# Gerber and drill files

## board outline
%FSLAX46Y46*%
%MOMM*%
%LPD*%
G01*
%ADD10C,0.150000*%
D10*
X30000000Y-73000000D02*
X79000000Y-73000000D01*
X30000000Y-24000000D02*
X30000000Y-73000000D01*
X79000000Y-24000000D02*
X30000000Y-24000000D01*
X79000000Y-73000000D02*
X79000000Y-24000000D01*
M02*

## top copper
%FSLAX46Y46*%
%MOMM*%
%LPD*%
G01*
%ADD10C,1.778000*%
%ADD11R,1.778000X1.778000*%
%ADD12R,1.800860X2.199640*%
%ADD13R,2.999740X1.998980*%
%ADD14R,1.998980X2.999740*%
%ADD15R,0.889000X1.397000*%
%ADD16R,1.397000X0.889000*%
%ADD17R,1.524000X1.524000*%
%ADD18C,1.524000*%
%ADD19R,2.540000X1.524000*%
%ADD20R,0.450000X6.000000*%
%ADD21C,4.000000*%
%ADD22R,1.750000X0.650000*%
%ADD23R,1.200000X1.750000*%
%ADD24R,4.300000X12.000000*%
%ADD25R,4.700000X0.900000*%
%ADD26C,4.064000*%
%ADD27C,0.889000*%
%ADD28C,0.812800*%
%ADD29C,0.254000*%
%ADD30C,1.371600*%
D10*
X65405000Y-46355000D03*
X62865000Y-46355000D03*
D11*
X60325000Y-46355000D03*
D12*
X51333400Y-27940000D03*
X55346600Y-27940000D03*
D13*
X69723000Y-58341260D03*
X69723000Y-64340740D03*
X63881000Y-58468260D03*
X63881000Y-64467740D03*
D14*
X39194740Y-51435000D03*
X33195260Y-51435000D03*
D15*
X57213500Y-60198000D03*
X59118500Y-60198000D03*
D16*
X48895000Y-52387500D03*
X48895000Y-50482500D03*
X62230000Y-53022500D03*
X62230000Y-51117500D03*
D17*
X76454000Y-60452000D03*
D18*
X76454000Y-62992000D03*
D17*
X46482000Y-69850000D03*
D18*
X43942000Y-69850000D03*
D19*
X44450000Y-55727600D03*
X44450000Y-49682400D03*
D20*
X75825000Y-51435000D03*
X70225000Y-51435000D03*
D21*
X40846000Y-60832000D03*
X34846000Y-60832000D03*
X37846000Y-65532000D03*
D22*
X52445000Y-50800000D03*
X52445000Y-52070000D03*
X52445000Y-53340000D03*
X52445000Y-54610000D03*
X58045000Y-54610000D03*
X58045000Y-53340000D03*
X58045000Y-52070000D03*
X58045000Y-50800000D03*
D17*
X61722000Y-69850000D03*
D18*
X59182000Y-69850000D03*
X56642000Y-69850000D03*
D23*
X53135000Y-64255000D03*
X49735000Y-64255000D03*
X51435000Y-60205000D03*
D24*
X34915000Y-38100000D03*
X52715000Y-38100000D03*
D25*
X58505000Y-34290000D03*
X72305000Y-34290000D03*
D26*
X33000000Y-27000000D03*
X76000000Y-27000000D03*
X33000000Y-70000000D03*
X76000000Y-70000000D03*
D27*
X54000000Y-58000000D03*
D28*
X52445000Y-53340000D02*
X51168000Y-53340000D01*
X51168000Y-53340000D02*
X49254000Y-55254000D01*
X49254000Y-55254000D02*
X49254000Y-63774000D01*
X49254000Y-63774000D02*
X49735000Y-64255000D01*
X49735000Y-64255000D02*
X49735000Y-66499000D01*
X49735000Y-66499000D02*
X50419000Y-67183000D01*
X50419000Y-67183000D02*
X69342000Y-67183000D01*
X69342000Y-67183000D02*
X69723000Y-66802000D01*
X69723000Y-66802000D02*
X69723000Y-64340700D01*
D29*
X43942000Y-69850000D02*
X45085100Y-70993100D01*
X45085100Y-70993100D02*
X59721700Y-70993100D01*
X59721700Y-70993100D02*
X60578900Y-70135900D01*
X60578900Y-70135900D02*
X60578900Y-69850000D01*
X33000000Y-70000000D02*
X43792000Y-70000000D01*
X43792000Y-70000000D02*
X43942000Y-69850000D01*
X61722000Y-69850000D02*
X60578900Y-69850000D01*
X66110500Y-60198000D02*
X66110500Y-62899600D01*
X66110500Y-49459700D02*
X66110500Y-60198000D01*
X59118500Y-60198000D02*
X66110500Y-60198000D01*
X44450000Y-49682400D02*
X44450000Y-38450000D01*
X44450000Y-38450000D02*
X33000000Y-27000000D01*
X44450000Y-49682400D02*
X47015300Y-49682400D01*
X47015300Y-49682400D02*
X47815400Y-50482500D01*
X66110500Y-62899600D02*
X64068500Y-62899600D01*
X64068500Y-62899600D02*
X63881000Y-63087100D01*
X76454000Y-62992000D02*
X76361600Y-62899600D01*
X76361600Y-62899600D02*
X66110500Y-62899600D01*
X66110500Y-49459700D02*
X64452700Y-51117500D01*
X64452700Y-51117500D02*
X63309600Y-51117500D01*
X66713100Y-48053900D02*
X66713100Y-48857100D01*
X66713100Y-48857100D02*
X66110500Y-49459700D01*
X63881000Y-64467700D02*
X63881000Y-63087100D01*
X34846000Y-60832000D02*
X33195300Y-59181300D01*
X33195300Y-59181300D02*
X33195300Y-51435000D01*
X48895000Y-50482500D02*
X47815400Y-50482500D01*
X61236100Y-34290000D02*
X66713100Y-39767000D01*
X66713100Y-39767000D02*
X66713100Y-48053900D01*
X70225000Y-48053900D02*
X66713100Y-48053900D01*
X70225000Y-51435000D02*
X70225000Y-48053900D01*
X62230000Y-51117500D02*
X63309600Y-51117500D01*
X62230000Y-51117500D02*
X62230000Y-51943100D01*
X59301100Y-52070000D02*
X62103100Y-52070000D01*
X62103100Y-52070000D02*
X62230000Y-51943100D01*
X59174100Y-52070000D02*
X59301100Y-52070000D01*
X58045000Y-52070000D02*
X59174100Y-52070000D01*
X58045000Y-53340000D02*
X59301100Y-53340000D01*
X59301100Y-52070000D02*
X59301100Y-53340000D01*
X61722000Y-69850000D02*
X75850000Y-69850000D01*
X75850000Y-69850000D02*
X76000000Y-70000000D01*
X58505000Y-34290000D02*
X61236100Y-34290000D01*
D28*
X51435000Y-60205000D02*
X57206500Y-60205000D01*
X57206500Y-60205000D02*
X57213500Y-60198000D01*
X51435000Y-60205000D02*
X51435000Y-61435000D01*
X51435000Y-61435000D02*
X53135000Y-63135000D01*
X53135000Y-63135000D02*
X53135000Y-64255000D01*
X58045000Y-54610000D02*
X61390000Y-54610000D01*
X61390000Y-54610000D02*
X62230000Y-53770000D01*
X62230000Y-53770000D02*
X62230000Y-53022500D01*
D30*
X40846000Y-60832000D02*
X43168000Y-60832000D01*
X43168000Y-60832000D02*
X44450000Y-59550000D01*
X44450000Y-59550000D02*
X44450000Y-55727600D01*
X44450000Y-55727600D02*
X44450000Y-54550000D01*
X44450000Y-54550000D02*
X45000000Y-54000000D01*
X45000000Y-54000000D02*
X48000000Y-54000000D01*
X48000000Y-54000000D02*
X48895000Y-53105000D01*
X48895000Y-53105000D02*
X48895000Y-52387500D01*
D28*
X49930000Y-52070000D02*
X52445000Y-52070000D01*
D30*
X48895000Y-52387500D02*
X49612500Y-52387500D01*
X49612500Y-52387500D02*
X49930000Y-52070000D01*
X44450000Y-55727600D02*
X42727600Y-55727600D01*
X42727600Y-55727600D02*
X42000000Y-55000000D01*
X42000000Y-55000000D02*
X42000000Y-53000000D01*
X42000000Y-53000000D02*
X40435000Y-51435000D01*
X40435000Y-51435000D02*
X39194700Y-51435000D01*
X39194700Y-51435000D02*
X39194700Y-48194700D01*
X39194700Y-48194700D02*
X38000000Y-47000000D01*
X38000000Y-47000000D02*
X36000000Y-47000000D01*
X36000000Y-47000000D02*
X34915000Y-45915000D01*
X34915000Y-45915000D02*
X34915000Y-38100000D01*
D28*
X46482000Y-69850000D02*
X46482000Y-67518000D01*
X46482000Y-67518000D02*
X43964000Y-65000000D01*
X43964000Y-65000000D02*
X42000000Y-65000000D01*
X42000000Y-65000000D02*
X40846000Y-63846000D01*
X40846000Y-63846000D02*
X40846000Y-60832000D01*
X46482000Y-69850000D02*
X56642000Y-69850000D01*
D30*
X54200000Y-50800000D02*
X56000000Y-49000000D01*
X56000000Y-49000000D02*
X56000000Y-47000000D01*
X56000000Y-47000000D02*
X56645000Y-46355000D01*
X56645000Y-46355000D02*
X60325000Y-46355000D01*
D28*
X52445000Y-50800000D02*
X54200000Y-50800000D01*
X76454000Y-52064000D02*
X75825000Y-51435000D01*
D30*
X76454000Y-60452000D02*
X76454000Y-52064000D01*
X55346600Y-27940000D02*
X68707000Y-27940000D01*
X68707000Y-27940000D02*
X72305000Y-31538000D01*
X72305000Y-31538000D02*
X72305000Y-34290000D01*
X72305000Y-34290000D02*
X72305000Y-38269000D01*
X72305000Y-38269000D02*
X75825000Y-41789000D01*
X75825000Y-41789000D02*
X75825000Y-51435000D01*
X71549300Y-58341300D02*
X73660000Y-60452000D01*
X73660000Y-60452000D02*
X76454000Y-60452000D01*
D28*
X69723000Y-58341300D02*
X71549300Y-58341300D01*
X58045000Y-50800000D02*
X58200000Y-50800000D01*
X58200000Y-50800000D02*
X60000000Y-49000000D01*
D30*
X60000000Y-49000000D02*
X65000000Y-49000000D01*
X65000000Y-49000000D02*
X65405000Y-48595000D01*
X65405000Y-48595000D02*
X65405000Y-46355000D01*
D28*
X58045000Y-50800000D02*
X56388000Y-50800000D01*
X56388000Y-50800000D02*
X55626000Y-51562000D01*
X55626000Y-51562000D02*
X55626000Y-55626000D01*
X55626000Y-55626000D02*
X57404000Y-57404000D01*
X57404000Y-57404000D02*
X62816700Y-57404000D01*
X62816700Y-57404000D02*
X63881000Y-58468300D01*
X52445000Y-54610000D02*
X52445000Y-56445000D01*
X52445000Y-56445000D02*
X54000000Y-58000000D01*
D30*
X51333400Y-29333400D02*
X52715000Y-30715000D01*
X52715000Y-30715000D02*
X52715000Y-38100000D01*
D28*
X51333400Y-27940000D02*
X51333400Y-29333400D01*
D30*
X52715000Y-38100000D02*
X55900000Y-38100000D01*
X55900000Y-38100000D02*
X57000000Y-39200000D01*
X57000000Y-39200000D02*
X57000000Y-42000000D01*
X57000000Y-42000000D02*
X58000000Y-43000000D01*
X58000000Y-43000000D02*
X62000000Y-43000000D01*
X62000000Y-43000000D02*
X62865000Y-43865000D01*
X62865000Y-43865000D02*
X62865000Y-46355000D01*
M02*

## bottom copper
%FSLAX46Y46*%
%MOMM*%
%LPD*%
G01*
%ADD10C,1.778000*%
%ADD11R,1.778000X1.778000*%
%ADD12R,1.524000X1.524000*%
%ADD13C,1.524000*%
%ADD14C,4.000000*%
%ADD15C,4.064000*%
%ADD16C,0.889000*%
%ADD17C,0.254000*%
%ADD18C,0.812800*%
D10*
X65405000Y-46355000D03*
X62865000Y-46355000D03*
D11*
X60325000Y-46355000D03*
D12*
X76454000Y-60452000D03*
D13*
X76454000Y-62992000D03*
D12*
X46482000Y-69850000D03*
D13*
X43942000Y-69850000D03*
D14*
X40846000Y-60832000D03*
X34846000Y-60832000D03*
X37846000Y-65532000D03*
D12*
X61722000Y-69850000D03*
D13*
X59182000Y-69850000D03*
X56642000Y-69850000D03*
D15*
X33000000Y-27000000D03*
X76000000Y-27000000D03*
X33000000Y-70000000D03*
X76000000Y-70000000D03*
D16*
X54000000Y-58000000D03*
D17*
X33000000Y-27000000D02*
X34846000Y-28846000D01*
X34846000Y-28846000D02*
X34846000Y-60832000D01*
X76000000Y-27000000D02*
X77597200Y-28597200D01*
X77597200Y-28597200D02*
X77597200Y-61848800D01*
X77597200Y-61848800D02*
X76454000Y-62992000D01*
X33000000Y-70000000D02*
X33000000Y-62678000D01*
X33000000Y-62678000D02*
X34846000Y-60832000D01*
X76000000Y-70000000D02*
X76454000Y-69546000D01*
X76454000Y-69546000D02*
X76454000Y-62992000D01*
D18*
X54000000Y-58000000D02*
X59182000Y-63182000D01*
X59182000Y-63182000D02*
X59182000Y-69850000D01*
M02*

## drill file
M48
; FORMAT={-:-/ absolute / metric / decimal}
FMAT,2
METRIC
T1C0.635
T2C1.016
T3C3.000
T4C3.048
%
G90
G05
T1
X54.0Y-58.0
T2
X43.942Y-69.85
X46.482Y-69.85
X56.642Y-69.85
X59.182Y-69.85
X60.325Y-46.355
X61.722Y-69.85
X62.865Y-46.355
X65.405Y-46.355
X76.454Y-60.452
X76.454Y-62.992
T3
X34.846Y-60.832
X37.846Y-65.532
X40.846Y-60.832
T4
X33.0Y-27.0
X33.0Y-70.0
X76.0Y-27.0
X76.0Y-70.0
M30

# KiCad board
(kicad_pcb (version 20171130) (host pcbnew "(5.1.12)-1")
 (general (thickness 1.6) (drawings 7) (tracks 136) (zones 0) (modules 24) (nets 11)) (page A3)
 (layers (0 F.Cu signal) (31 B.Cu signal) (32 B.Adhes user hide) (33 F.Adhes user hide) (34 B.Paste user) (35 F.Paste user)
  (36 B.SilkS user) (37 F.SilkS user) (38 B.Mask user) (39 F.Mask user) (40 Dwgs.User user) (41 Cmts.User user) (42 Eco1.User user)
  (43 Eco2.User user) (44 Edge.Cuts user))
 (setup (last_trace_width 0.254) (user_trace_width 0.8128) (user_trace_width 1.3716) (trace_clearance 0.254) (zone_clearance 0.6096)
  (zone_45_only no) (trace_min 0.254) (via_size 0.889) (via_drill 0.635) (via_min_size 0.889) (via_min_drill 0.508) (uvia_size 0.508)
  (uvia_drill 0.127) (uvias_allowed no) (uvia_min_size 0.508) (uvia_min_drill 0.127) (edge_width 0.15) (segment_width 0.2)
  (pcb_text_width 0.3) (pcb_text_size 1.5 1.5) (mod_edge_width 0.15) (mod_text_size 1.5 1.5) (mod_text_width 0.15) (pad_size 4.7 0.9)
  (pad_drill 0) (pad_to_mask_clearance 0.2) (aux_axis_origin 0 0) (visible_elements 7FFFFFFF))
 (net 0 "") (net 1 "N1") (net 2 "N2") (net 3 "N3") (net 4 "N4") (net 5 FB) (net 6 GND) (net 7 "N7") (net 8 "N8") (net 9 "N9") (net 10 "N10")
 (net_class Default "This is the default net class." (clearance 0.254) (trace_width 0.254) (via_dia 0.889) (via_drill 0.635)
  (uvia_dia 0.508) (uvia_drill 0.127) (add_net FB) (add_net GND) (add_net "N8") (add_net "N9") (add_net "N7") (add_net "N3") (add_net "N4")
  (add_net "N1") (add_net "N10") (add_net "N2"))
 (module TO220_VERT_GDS (layer F.Cu) (at 62.865 46.355 270)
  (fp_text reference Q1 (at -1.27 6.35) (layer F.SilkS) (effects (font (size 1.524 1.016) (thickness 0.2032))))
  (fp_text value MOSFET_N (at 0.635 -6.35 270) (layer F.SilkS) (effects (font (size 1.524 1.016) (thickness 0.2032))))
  (pad S thru_hole circle (at 0 -2.54 270) (size 1.778 1.778) (drill 1.016) (layers *.Cu *.Mask F.SilkS) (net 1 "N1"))
  (pad D thru_hole circle (at 0 0 270) (size 1.778 1.778) (drill 1.016) (layers *.Cu *.Mask F.SilkS) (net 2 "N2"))
  (pad G thru_hole rect (at 0 2.54 270) (size 1.778 1.778) (drill 1.016) (layers *.Cu *.Mask F.SilkS) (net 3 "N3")))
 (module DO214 (layer F.Cu) (at 53.34 27.94)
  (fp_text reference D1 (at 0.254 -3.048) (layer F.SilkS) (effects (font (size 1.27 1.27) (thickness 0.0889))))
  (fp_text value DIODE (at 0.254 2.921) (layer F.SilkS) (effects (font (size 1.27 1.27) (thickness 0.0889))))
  (pad 1 smd rect (at -2.0066 0) (size 1.80086 2.19964) (layers F.Cu F.Paste F.Mask) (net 2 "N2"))
  (pad 2 smd rect (at 2.0066 0) (size 1.80086 2.19964) (layers F.Cu F.Paste F.Mask) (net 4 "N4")))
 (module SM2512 (layer F.Cu) (at 69.723 61.341 270)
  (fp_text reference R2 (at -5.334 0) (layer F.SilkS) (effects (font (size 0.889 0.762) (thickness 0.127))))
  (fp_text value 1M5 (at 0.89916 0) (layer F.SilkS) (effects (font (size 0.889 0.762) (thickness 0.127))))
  (pad 1 smd rect (at -2.99974 0 270) (size 1.99898 2.99974) (layers F.Cu F.Paste F.Mask) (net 4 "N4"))
  (pad 2 smd rect (at 2.99974 0 270) (size 1.99898 2.99974) (layers F.Cu F.Paste F.Mask) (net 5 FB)))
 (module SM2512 (layer F.Cu) (at 63.881 61.468 270)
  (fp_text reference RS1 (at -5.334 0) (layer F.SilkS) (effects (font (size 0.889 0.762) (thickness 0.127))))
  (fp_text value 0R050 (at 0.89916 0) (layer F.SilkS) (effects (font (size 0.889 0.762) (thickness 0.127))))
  (pad 1 smd rect (at -2.99974 0 270) (size 1.99898 2.99974) (layers F.Cu F.Paste F.Mask) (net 1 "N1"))
  (pad 2 smd rect (at 2.99974 0 270) (size 1.99898 2.99974) (layers F.Cu F.Paste F.Mask) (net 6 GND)))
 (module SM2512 (layer F.Cu) (at 36.195 51.435 180)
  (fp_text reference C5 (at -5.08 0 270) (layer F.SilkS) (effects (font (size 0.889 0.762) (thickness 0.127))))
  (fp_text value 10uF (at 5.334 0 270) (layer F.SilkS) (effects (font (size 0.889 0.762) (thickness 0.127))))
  (pad 1 smd rect (at -2.99974 0 180) (size 1.99898 2.99974) (layers F.Cu F.Paste F.Mask) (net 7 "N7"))
  (pad 2 smd rect (at 2.99974 0 180) (size 1.99898 2.99974) (layers F.Cu F.Paste F.Mask) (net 6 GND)))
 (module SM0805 (layer F.Cu) (at 58.166 60.198)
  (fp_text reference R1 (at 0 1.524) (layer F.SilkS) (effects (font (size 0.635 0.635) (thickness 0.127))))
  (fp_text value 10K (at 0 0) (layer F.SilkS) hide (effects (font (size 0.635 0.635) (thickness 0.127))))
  (pad 1 smd rect (at -0.9525 0) (size 0.889 1.397) (layers F.Cu F.Paste F.Mask) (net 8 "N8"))
  (pad 2 smd rect (at 0.9525 0) (size 0.889 1.397) (layers F.Cu F.Paste F.Mask) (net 6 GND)))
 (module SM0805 (layer F.Cu) (at 48.895 51.435 90)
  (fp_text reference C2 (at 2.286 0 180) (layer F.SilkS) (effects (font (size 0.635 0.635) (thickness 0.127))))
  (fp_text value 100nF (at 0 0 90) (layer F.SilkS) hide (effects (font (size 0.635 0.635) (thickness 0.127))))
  (pad 1 smd rect (at -0.9525 0 90) (size 0.889 1.397) (layers F.Cu F.Paste F.Mask) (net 7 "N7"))
  (pad 2 smd rect (at 0.9525 0 90) (size 0.889 1.397) (layers F.Cu F.Paste F.Mask) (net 6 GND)))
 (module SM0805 (layer F.Cu) (at 62.23 52.07 90)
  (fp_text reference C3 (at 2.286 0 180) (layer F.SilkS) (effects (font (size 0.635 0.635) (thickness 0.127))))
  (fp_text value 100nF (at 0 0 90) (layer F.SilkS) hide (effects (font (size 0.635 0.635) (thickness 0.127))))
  (pad 1 smd rect (at -0.9525 0 90) (size 0.889 1.397) (layers F.Cu F.Paste F.Mask) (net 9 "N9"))
  (pad 2 smd rect (at 0.9525 0 90) (size 0.889 1.397) (layers F.Cu F.Paste F.Mask) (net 6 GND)))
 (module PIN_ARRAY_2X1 (layer F.Cu) (at 76.454 61.722 270)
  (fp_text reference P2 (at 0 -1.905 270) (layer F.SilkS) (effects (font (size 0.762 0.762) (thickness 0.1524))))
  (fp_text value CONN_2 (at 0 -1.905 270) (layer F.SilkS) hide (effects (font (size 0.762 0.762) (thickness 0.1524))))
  (pad 1 thru_hole rect (at -1.27 0 270) (size 1.524 1.524) (drill 1.016) (layers *.Cu *.Mask F.SilkS) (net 4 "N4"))
  (pad 2 thru_hole circle (at 1.27 0 270) (size 1.524 1.524) (drill 1.016) (layers *.Cu *.Mask F.SilkS) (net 6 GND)))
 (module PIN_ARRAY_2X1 (layer F.Cu) (at 45.212 69.85 180)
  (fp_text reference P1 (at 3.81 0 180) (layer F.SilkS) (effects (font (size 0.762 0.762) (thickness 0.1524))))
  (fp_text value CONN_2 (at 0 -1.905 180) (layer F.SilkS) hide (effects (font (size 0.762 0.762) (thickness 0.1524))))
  (pad 1 thru_hole rect (at -1.27 0 180) (size 1.524 1.524) (drill 1.016) (layers *.Cu *.Mask F.SilkS) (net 7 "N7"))
  (pad 2 thru_hole circle (at 1.27 0 180) (size 1.524 1.524) (drill 1.016) (layers *.Cu *.Mask F.SilkS) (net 6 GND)))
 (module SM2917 (layer F.Cu) (at 44.45 52.705 90)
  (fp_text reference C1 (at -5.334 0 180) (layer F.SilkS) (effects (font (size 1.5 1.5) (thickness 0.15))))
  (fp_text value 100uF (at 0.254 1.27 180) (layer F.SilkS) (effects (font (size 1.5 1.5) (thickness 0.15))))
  (pad 1 smd rect (at -3.0226 0 90) (size 1.524 2.54) (layers F.Cu F.Paste F.Mask) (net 7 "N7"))
  (pad 2 smd rect (at 3.0226 0 90) (size 1.524 2.54) (layers F.Cu F.Paste F.Mask) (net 6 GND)))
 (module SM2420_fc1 (layer F.Cu) (at 73.025 51.435 180)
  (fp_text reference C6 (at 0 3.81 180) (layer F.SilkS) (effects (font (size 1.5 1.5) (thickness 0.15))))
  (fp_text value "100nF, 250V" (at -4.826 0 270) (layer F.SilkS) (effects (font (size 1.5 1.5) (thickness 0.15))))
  (pad 1 smd rect (at -2.8 0 180) (size 0.45 6) (layers F.Cu F.Paste F.Mask) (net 4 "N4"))
  (pad 2 smd rect (at 2.8 0 180) (size 0.45 6) (layers F.Cu F.Paste F.Mask) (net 6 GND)))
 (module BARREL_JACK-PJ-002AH (layer F.Cu) (at 37.846 65.532 180)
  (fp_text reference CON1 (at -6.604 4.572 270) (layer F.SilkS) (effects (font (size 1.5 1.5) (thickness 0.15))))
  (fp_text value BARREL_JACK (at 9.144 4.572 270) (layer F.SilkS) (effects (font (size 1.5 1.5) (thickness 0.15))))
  (pad 1 thru_hole circle (at -3 4.7 180) (size 4 4) (drill 3) (layers *.Cu *.Mask F.SilkS) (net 7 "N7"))
  (pad 2 thru_hole circle (at 3 4.7 180) (size 4 4) (drill 3) (layers *.Cu *.Mask F.SilkS) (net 6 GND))
  (pad 3 thru_hole circle (at 0 0 180) (size 4 4) (drill 3) (layers *.Cu *.Mask F.SilkS)))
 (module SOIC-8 (layer F.Cu) (at 55.245 52.705 270)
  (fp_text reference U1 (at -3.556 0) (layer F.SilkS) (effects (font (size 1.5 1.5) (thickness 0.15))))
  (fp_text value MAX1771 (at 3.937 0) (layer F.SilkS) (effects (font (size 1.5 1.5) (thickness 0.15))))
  (pad 1 smd rect (at -1.905 2.8 270) (size 0.65 1.75) (layers F.Cu F.Paste F.Mask) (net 3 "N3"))
  (pad 2 smd rect (at -0.635 2.8 270) (size 0.65 1.75) (layers F.Cu F.Paste F.Mask) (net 7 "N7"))
  (pad 3 smd rect (at 0.635 2.8 270) (size 0.65 1.75) (layers F.Cu F.Paste F.Mask) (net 5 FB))
  (pad 4 smd rect (at 1.905 2.8 270) (size 0.65 1.75) (layers F.Cu F.Paste F.Mask) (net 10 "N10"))
  (pad 5 smd rect (at 1.905 -2.8 270) (size 0.65 1.75) (layers F.Cu F.Paste F.Mask) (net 9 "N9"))
  (pad 6 smd rect (at 0.635 -2.8 270) (size 0.65 1.75) (layers F.Cu F.Paste F.Mask) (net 6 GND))
  (pad 7 smd rect (at -0.635 -2.8 270) (size 0.65 1.75) (layers F.Cu F.Paste F.Mask) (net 6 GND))
  (pad 8 smd rect (at -1.905 -2.8 270) (size 0.65 1.75) (layers F.Cu F.Paste F.Mask) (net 1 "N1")))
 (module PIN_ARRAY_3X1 (layer F.Cu) (at 59.182 69.85 180)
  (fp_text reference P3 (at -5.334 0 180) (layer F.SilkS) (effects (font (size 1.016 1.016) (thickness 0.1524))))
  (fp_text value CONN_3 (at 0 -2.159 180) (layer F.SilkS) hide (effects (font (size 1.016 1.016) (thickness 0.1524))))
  (pad 1 thru_hole rect (at -2.54 0 180) (size 1.524 1.524) (drill 1.016) (layers *.Cu *.Mask F.SilkS) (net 6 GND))
  (pad 2 thru_hole circle (at 0 0 180) (size 1.524 1.524) (drill 1.016) (layers *.Cu *.Mask F.SilkS) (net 10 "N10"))
  (pad 3 thru_hole circle (at 2.54 0 180) (size 1.524 1.524) (drill 1.016) (layers *.Cu *.Mask F.SilkS) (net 7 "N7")))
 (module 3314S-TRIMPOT (layer F.Cu) (at 51.435 62.23 180)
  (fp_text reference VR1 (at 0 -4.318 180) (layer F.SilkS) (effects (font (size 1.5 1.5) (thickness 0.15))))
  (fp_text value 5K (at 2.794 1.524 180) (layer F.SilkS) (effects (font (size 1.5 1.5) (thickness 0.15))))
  (pad 3 smd rect (at -1.7 -2.025 180) (size 1.2 1.75) (layers F.Cu F.Paste F.Mask) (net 8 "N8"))
  (pad 1 smd rect (at 1.7 -2.025 180) (size 1.2 1.75) (layers F.Cu F.Paste F.Mask) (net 5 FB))
  (pad 2 smd rect (at 0 2.025 180) (size 1.2 1.75) (layers F.Cu F.Paste F.Mask) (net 8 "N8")))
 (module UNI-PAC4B (layer F.Cu) (at 43.815 38.1)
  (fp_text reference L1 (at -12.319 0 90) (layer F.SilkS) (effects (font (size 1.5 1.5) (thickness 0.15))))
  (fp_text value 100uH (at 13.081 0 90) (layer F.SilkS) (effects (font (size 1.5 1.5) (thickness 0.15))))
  (pad 1 smd rect (at -8.9 0) (size 4.3 12) (layers F.Cu F.Paste F.Mask) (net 7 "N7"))
  (pad 2 smd rect (at 8.9 0) (size 4.3 12) (layers F.Cu F.Paste F.Mask) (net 2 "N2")))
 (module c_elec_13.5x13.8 (layer F.Cu) (at 65.405 34.29)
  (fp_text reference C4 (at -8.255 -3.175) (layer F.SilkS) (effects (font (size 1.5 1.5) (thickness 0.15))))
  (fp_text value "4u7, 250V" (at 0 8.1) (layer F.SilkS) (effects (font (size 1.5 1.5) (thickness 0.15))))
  (pad 2 smd rect (at -6.9 0) (size 4.7 0.9) (layers F.Cu F.Paste F.Mask) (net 6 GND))
  (pad 1 smd rect (at 6.9 0) (size 4.7 0.9) (layers F.Cu F.Paste F.Mask) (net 4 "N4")))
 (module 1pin (layer F.Cu) (at 33 27)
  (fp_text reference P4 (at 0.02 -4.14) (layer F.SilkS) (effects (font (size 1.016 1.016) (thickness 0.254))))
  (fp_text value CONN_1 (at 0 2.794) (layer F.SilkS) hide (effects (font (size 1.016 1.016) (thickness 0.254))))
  (pad 1 thru_hole circle (at 0 0) (size 4.064 4.064) (drill 3.048) (layers *.Cu *.Mask F.SilkS) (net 6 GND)))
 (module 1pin (layer F.Cu) (at 76 27)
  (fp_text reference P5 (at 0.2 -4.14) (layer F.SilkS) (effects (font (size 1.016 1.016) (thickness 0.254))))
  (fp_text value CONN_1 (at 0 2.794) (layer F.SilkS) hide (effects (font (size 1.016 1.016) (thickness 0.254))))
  (pad 1 thru_hole circle (at 0 0) (size 4.064 4.064) (drill 3.048) (layers *.Cu *.Mask F.SilkS) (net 6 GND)))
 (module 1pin (layer F.Cu) (at 33 70)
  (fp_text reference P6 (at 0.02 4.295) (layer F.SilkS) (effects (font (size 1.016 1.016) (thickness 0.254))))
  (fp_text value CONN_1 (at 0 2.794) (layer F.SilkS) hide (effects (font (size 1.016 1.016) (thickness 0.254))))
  (pad 1 thru_hole circle (at 0 0) (size 4.064 4.064) (drill 3.048) (layers *.Cu *.Mask F.SilkS) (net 6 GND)))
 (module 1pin (layer F.Cu) (at 76 70)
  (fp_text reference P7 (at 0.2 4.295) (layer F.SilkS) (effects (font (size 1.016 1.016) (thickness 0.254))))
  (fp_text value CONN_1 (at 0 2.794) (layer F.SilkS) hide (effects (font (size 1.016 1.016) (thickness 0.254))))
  (pad 1 thru_hole circle (at 0 0) (size 4.064 4.064) (drill 3.048) (layers *.Cu *.Mask F.SilkS) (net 6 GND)))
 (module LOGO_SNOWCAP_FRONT (layer F.Cu) (at 53 65)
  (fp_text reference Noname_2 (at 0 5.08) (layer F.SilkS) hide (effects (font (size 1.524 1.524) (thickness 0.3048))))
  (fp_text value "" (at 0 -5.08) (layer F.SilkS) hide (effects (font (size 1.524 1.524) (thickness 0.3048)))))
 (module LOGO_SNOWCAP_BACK (layer B.Cu) (at 53 51)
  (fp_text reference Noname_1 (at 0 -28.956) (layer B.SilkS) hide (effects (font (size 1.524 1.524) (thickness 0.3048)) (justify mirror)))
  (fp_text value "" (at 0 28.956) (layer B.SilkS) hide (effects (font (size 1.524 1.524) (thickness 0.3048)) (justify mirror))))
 (gr_line (start 30 73) (end 79 73) (angle 90) (layer Edge.Cuts) (width 0.15))
 (gr_line (start 30 24) (end 30 73) (angle 90) (layer Edge.Cuts) (width 0.15))
 (gr_line (start 79 24) (end 30 24) (angle 90) (layer Edge.Cuts) (width 0.15))
 (gr_line (start 79 73) (end 79 24) (angle 90) (layer Edge.Cuts) (width 0.15))
 (segment (start 52.445 53.34) (end 51.168 53.34) (width 0.8128) (layer F.Cu) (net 5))
 (segment (start 51.168 53.34) (end 49.254 55.254) (width 0.8128) (layer F.Cu) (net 5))
 (segment (start 49.254 55.254) (end 49.254 63.774) (width 0.8128) (layer F.Cu) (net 5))
 (segment (start 49.254 63.774) (end 49.735 64.255) (width 0.8128) (layer F.Cu) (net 5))
 (segment (start 49.735 64.255) (end 49.735 66.499) (width 0.8128) (layer F.Cu) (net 5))
 (segment (start 49.735 66.499) (end 50.419 67.183) (width 0.8128) (layer F.Cu) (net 5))
 (segment (start 50.419 67.183) (end 69.342 67.183) (width 0.8128) (layer F.Cu) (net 5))
 (segment (start 69.342 67.183) (end 69.723 66.802) (width 0.8128) (layer F.Cu) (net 5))
 (segment (start 69.723 66.802) (end 69.723 64.3407) (width 0.8128) (layer F.Cu) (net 5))
 (segment (start 43.942 69.85) (end 45.0851 70.9931) (width 0.254) (layer F.Cu) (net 6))
 (segment (start 45.0851 70.9931) (end 59.7217 70.9931) (width 0.254) (layer F.Cu) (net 6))
 (segment (start 59.7217 70.9931) (end 60.5789 70.1359) (width 0.254) (layer F.Cu) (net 6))
 (segment (start 60.5789 70.1359) (end 60.5789 69.85) (width 0.254) (layer F.Cu) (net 6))
 (segment (start 33 70) (end 43.792 70) (width 0.254) (layer F.Cu) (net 6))
 (segment (start 43.792 70) (end 43.942 69.85) (width 0.254) (layer F.Cu) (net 6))
 (segment (start 61.722 69.85) (end 60.5789 69.85) (width 0.254) (layer F.Cu) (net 6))
 (segment (start 66.1105 60.198) (end 66.1105 62.8996) (width 0.254) (layer F.Cu) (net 6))
 (segment (start 66.1105 49.4597) (end 66.1105 60.198) (width 0.254) (layer F.Cu) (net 6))
 (segment (start 59.1185 60.198) (end 66.1105 60.198) (width 0.254) (layer F.Cu) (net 6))
 (segment (start 44.45 49.6824) (end 44.45 38.45) (width 0.254) (layer F.Cu) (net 6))
 (segment (start 44.45 38.45) (end 33 27) (width 0.254) (layer F.Cu) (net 6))
 (segment (start 44.45 49.6824) (end 47.0153 49.6824) (width 0.254) (layer F.Cu) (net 6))
 (segment (start 47.0153 49.6824) (end 47.8154 50.4825) (width 0.254) (layer F.Cu) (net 6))
 (segment (start 66.1105 62.8996) (end 64.0685 62.8996) (width 0.254) (layer F.Cu) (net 6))
 (segment (start 64.0685 62.8996) (end 63.881 63.0871) (width 0.254) (layer F.Cu) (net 6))
 (segment (start 76.454 62.992) (end 76.3616 62.8996) (width 0.254) (layer F.Cu) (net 6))
 (segment (start 76.3616 62.8996) (end 66.1105 62.8996) (width 0.254) (layer F.Cu) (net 6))
 (segment (start 66.1105 49.4597) (end 64.4527 51.1175) (width 0.254) (layer F.Cu) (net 6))
 (segment (start 64.4527 51.1175) (end 63.3096 51.1175) (width 0.254) (layer F.Cu) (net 6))
 (segment (start 66.7131 48.0539) (end 66.7131 48.8571) (width 0.254) (layer F.Cu) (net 6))
 (segment (start 66.7131 48.8571) (end 66.1105 49.4597) (width 0.254) (layer F.Cu) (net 6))
 (segment (start 63.881 64.4677) (end 63.881 63.0871) (width 0.254) (layer F.Cu) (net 6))
 (segment (start 34.846 60.832) (end 33.1953 59.1813) (width 0.254) (layer F.Cu) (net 6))
 (segment (start 33.1953 59.1813) (end 33.1953 51.435) (width 0.254) (layer F.Cu) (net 6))
 (segment (start 48.895 50.4825) (end 47.8154 50.4825) (width 0.254) (layer F.Cu) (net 6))
 (segment (start 61.2361 34.29) (end 66.7131 39.767) (width 0.254) (layer F.Cu) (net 6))
 (segment (start 66.7131 39.767) (end 66.7131 48.0539) (width 0.254) (layer F.Cu) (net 6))
 (segment (start 70.225 48.0539) (end 66.7131 48.0539) (width 0.254) (layer F.Cu) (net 6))
 (segment (start 70.225 51.435) (end 70.225 48.0539) (width 0.254) (layer F.Cu) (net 6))
 (segment (start 62.23 51.1175) (end 63.3096 51.1175) (width 0.254) (layer F.Cu) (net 6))
 (segment (start 62.23 51.1175) (end 62.23 51.9431) (width 0.254) (layer F.Cu) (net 6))
 (segment (start 59.3011 52.07) (end 62.1031 52.07) (width 0.254) (layer F.Cu) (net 6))
 (segment (start 62.1031 52.07) (end 62.23 51.9431) (width 0.254) (layer F.Cu) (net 6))
 (segment (start 59.1741 52.07) (end 59.3011 52.07) (width 0.254) (layer F.Cu) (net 6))
 (segment (start 58.045 52.07) (end 59.1741 52.07) (width 0.254) (layer F.Cu) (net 6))
 (segment (start 58.045 53.34) (end 59.3011 53.34) (width 0.254) (layer F.Cu) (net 6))
 (segment (start 59.3011 52.07) (end 59.3011 53.34) (width 0.254) (layer F.Cu) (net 6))
 (segment (start 61.722 69.85) (end 75.85 69.85) (width 0.254) (layer F.Cu) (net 6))
 (segment (start 75.85 69.85) (end 76 70) (width 0.254) (layer F.Cu) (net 6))
 (segment (start 58.505 34.29) (end 61.2361 34.29) (width 0.254) (layer F.Cu) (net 6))
 (segment (start 33 27) (end 34.846 28.846) (width 0.254) (layer B.Cu) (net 6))
 (segment (start 34.846 28.846) (end 34.846 60.832) (width 0.254) (layer B.Cu) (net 6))
 (segment (start 76 27) (end 77.5972 28.5972) (width 0.254) (layer B.Cu) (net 6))
 (segment (start 77.5972 28.5972) (end 77.5972 61.8488) (width 0.254) (layer B.Cu) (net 6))
 (segment (start 77.5972 61.8488) (end 76.454 62.992) (width 0.254) (layer B.Cu) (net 6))
 (segment (start 33 70) (end 33 62.678) (width 0.254) (layer B.Cu) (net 6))
 (segment (start 33 62.678) (end 34.846 60.832) (width 0.254) (layer B.Cu) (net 6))
 (segment (start 76 70) (end 76.454 69.546) (width 0.254) (layer B.Cu) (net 6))
 (segment (start 76.454 69.546) (end 76.454 62.992) (width 0.254) (layer B.Cu) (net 6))
 (segment (start 51.435 60.205) (end 57.2065 60.205) (width 0.8128) (layer F.Cu) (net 8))
 (segment (start 57.2065 60.205) (end 57.2135 60.198) (width 0.8128) (layer F.Cu) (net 8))
 (segment (start 51.435 60.205) (end 51.435 61.435) (width 0.8128) (layer F.Cu) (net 8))
 (segment (start 51.435 61.435) (end 53.135 63.135) (width 0.8128) (layer F.Cu) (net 8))
 (segment (start 53.135 63.135) (end 53.135 64.255) (width 0.8128) (layer F.Cu) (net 8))
 (segment (start 58.045 54.61) (end 61.39 54.61) (width 0.8128) (layer F.Cu) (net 9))
 (segment (start 61.39 54.61) (end 62.23 53.77) (width 0.8128) (layer F.Cu) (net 9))
 (segment (start 62.23 53.77) (end 62.23 53.0225) (width 0.8128) (layer F.Cu) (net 9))
 (segment (start 40.846 60.832) (end 43.168 60.832) (width 1.3716) (layer F.Cu) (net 7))
 (segment (start 43.168 60.832) (end 44.45 59.55) (width 1.3716) (layer F.Cu) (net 7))
 (segment (start 44.45 59.55) (end 44.45 55.7276) (width 1.3716) (layer F.Cu) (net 7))
 (segment (start 44.45 55.7276) (end 44.45 54.55) (width 1.3716) (layer F.Cu) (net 7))
 (segment (start 44.45 54.55) (end 45 54) (width 1.3716) (layer F.Cu) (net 7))
 (segment (start 45 54) (end 48 54) (width 1.3716) (layer F.Cu) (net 7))
 (segment (start 48 54) (end 48.895 53.105) (width 1.3716) (layer F.Cu) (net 7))
 (segment (start 48.895 53.105) (end 48.895 52.3875) (width 1.3716) (layer F.Cu) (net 7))
 (segment (start 49.93 52.07) (end 52.445 52.07) (width 0.8128) (layer F.Cu) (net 7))
 (segment (start 48.895 52.3875) (end 49.6125 52.3875) (width 1.3716) (layer F.Cu) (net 7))
 (segment (start 49.6125 52.3875) (end 49.93 52.07) (width 1.3716) (layer F.Cu) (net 7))
 (segment (start 44.45 55.7276) (end 42.7276 55.7276) (width 1.3716) (layer F.Cu) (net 7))
 (segment (start 42.7276 55.7276) (end 42 55) (width 1.3716) (layer F.Cu) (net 7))
 (segment (start 42 55) (end 42 53) (width 1.3716) (layer F.Cu) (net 7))
 (segment (start 42 53) (end 40.435 51.435) (width 1.3716) (layer F.Cu) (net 7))
 (segment (start 40.435 51.435) (end 39.1947 51.435) (width 1.3716) (layer F.Cu) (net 7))
 (segment (start 39.1947 51.435) (end 39.1947 48.1947) (width 1.3716) (layer F.Cu) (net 7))
 (segment (start 39.1947 48.1947) (end 38 47) (width 1.3716) (layer F.Cu) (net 7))
 (segment (start 38 47) (end 36 47) (width 1.3716) (layer F.Cu) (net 7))
 (segment (start 36 47) (end 34.915 45.915) (width 1.3716) (layer F.Cu) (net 7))
 (segment (start 34.915 45.915) (end 34.915 38.1) (width 1.3716) (layer F.Cu) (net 7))
 (segment (start 46.482 69.85) (end 46.482 67.518) (width 0.8128) (layer F.Cu) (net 7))
 (segment (start 46.482 67.518) (end 43.964 65) (width 0.8128) (layer F.Cu) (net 7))
 (segment (start 43.964 65) (end 42 65) (width 0.8128) (layer F.Cu) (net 7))
 (segment (start 42 65) (end 40.846 63.846) (width 0.8128) (layer F.Cu) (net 7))
 (segment (start 40.846 63.846) (end 40.846 60.832) (width 0.8128) (layer F.Cu) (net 7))
 (segment (start 46.482 69.85) (end 56.642 69.85) (width 0.8128) (layer F.Cu) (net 7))
 (segment (start 54.2 50.8) (end 56 49) (width 1.3716) (layer F.Cu) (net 3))
 (segment (start 56 49) (end 56 47) (width 1.3716) (layer F.Cu) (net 3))
 (segment (start 56 47) (end 56.645 46.355) (width 1.3716) (layer F.Cu) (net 3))
 (segment (start 56.645 46.355) (end 60.325 46.355) (width 1.3716) (layer F.Cu) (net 3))
 (segment (start 52.445 50.8) (end 54.2 50.8) (width 0.8128) (layer F.Cu) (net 3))
 (segment (start 76.454 52.064) (end 75.825 51.435) (width 0.8128) (layer F.Cu) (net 4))
 (segment (start 76.454 60.452) (end 76.454 52.064) (width 1.3716) (layer F.Cu) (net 4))
 (segment (start 55.3466 27.94) (end 68.707 27.94) (width 1.3716) (layer F.Cu) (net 4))
 (segment (start 68.707 27.94) (end 72.305 31.538) (width 1.3716) (layer F.Cu) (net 4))
 (segment (start 72.305 31.538) (end 72.305 34.29) (width 1.3716) (layer F.Cu) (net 4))
 (segment (start 72.305 34.29) (end 72.305 38.269) (width 1.3716) (layer F.Cu) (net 4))
 (segment (start 72.305 38.269) (end 75.825 41.789) (width 1.3716) (layer F.Cu) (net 4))
 (segment (start 75.825 41.789) (end 75.825 51.435) (width 1.3716) (layer F.Cu) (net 4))
 (segment (start 71.5493 58.3413) (end 73.66 60.452) (width 1.3716) (layer F.Cu) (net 4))
 (segment (start 73.66 60.452) (end 76.454 60.452) (width 1.3716) (layer F.Cu) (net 4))
 (segment (start 69.723 58.3413) (end 71.5493 58.3413) (width 0.8128) (layer F.Cu) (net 4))
 (segment (start 58.045 50.8) (end 58.2 50.8) (width 0.8128) (layer F.Cu) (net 1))
 (segment (start 58.2 50.8) (end 60 49) (width 0.8128) (layer F.Cu) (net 1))
 (segment (start 60 49) (end 65 49) (width 1.3716) (layer F.Cu) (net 1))
 (segment (start 65 49) (end 65.405 48.595) (width 1.3716) (layer F.Cu) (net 1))
 (segment (start 65.405 48.595) (end 65.405 46.355) (width 1.3716) (layer F.Cu) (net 1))
 (segment (start 58.045 50.8) (end 56.388 50.8) (width 0.8128) (layer F.Cu) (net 1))
 (segment (start 56.388 50.8) (end 55.626 51.562) (width 0.8128) (layer F.Cu) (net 1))
 (segment (start 55.626 51.562) (end 55.626 55.626) (width 0.8128) (layer F.Cu) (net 1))
 (segment (start 55.626 55.626) (end 57.404 57.404) (width 0.8128) (layer F.Cu) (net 1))
 (segment (start 57.404 57.404) (end 62.8167 57.404) (width 0.8128) (layer F.Cu) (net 1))
 (segment (start 62.8167 57.404) (end 63.881 58.4683) (width 0.8128) (layer F.Cu) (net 1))
 (segment (start 52.445 54.61) (end 52.445 56.445) (width 0.8128) (layer F.Cu) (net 10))
 (segment (start 52.445 56.445) (end 54 58) (width 0.8128) (layer F.Cu) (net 10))
 (segment (start 54 58) (end 59.182 63.182) (width 0.8128) (layer B.Cu) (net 10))
 (segment (start 59.182 63.182) (end 59.182 69.85) (width 0.8128) (layer B.Cu) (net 10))
 (via (at 54 58) (size 0.889) (layers F.Cu B.Cu) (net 10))
 (segment (start 51.3334 29.3334) (end 52.715 30.715) (width 1.3716) (layer F.Cu) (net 2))
 (segment (start 52.715 30.715) (end 52.715 38.1) (width 1.3716) (layer F.Cu) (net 2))
 (segment (start 51.3334 27.94) (end 51.3334 29.3334) (width 0.8128) (layer F.Cu) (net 2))
 (segment (start 52.715 38.1) (end 55.9 38.1) (width 1.3716) (layer F.Cu) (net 2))
 (segment (start 55.9 38.1) (end 57 39.2) (width 1.3716) (layer F.Cu) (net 2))
 (segment (start 57 39.2) (end 57 42) (width 1.3716) (layer F.Cu) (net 2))
 (segment (start 57 42) (end 58 43) (width 1.3716) (layer F.Cu) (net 2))
 (segment (start 58 43) (end 62 43) (width 1.3716) (layer F.Cu) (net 2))
 (segment (start 62 43) (end 62.865 43.865) (width 1.3716) (layer F.Cu) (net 2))
 (segment (start 62.865 43.865) (end 62.865 46.355) (width 1.3716) (layer F.Cu) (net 2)))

